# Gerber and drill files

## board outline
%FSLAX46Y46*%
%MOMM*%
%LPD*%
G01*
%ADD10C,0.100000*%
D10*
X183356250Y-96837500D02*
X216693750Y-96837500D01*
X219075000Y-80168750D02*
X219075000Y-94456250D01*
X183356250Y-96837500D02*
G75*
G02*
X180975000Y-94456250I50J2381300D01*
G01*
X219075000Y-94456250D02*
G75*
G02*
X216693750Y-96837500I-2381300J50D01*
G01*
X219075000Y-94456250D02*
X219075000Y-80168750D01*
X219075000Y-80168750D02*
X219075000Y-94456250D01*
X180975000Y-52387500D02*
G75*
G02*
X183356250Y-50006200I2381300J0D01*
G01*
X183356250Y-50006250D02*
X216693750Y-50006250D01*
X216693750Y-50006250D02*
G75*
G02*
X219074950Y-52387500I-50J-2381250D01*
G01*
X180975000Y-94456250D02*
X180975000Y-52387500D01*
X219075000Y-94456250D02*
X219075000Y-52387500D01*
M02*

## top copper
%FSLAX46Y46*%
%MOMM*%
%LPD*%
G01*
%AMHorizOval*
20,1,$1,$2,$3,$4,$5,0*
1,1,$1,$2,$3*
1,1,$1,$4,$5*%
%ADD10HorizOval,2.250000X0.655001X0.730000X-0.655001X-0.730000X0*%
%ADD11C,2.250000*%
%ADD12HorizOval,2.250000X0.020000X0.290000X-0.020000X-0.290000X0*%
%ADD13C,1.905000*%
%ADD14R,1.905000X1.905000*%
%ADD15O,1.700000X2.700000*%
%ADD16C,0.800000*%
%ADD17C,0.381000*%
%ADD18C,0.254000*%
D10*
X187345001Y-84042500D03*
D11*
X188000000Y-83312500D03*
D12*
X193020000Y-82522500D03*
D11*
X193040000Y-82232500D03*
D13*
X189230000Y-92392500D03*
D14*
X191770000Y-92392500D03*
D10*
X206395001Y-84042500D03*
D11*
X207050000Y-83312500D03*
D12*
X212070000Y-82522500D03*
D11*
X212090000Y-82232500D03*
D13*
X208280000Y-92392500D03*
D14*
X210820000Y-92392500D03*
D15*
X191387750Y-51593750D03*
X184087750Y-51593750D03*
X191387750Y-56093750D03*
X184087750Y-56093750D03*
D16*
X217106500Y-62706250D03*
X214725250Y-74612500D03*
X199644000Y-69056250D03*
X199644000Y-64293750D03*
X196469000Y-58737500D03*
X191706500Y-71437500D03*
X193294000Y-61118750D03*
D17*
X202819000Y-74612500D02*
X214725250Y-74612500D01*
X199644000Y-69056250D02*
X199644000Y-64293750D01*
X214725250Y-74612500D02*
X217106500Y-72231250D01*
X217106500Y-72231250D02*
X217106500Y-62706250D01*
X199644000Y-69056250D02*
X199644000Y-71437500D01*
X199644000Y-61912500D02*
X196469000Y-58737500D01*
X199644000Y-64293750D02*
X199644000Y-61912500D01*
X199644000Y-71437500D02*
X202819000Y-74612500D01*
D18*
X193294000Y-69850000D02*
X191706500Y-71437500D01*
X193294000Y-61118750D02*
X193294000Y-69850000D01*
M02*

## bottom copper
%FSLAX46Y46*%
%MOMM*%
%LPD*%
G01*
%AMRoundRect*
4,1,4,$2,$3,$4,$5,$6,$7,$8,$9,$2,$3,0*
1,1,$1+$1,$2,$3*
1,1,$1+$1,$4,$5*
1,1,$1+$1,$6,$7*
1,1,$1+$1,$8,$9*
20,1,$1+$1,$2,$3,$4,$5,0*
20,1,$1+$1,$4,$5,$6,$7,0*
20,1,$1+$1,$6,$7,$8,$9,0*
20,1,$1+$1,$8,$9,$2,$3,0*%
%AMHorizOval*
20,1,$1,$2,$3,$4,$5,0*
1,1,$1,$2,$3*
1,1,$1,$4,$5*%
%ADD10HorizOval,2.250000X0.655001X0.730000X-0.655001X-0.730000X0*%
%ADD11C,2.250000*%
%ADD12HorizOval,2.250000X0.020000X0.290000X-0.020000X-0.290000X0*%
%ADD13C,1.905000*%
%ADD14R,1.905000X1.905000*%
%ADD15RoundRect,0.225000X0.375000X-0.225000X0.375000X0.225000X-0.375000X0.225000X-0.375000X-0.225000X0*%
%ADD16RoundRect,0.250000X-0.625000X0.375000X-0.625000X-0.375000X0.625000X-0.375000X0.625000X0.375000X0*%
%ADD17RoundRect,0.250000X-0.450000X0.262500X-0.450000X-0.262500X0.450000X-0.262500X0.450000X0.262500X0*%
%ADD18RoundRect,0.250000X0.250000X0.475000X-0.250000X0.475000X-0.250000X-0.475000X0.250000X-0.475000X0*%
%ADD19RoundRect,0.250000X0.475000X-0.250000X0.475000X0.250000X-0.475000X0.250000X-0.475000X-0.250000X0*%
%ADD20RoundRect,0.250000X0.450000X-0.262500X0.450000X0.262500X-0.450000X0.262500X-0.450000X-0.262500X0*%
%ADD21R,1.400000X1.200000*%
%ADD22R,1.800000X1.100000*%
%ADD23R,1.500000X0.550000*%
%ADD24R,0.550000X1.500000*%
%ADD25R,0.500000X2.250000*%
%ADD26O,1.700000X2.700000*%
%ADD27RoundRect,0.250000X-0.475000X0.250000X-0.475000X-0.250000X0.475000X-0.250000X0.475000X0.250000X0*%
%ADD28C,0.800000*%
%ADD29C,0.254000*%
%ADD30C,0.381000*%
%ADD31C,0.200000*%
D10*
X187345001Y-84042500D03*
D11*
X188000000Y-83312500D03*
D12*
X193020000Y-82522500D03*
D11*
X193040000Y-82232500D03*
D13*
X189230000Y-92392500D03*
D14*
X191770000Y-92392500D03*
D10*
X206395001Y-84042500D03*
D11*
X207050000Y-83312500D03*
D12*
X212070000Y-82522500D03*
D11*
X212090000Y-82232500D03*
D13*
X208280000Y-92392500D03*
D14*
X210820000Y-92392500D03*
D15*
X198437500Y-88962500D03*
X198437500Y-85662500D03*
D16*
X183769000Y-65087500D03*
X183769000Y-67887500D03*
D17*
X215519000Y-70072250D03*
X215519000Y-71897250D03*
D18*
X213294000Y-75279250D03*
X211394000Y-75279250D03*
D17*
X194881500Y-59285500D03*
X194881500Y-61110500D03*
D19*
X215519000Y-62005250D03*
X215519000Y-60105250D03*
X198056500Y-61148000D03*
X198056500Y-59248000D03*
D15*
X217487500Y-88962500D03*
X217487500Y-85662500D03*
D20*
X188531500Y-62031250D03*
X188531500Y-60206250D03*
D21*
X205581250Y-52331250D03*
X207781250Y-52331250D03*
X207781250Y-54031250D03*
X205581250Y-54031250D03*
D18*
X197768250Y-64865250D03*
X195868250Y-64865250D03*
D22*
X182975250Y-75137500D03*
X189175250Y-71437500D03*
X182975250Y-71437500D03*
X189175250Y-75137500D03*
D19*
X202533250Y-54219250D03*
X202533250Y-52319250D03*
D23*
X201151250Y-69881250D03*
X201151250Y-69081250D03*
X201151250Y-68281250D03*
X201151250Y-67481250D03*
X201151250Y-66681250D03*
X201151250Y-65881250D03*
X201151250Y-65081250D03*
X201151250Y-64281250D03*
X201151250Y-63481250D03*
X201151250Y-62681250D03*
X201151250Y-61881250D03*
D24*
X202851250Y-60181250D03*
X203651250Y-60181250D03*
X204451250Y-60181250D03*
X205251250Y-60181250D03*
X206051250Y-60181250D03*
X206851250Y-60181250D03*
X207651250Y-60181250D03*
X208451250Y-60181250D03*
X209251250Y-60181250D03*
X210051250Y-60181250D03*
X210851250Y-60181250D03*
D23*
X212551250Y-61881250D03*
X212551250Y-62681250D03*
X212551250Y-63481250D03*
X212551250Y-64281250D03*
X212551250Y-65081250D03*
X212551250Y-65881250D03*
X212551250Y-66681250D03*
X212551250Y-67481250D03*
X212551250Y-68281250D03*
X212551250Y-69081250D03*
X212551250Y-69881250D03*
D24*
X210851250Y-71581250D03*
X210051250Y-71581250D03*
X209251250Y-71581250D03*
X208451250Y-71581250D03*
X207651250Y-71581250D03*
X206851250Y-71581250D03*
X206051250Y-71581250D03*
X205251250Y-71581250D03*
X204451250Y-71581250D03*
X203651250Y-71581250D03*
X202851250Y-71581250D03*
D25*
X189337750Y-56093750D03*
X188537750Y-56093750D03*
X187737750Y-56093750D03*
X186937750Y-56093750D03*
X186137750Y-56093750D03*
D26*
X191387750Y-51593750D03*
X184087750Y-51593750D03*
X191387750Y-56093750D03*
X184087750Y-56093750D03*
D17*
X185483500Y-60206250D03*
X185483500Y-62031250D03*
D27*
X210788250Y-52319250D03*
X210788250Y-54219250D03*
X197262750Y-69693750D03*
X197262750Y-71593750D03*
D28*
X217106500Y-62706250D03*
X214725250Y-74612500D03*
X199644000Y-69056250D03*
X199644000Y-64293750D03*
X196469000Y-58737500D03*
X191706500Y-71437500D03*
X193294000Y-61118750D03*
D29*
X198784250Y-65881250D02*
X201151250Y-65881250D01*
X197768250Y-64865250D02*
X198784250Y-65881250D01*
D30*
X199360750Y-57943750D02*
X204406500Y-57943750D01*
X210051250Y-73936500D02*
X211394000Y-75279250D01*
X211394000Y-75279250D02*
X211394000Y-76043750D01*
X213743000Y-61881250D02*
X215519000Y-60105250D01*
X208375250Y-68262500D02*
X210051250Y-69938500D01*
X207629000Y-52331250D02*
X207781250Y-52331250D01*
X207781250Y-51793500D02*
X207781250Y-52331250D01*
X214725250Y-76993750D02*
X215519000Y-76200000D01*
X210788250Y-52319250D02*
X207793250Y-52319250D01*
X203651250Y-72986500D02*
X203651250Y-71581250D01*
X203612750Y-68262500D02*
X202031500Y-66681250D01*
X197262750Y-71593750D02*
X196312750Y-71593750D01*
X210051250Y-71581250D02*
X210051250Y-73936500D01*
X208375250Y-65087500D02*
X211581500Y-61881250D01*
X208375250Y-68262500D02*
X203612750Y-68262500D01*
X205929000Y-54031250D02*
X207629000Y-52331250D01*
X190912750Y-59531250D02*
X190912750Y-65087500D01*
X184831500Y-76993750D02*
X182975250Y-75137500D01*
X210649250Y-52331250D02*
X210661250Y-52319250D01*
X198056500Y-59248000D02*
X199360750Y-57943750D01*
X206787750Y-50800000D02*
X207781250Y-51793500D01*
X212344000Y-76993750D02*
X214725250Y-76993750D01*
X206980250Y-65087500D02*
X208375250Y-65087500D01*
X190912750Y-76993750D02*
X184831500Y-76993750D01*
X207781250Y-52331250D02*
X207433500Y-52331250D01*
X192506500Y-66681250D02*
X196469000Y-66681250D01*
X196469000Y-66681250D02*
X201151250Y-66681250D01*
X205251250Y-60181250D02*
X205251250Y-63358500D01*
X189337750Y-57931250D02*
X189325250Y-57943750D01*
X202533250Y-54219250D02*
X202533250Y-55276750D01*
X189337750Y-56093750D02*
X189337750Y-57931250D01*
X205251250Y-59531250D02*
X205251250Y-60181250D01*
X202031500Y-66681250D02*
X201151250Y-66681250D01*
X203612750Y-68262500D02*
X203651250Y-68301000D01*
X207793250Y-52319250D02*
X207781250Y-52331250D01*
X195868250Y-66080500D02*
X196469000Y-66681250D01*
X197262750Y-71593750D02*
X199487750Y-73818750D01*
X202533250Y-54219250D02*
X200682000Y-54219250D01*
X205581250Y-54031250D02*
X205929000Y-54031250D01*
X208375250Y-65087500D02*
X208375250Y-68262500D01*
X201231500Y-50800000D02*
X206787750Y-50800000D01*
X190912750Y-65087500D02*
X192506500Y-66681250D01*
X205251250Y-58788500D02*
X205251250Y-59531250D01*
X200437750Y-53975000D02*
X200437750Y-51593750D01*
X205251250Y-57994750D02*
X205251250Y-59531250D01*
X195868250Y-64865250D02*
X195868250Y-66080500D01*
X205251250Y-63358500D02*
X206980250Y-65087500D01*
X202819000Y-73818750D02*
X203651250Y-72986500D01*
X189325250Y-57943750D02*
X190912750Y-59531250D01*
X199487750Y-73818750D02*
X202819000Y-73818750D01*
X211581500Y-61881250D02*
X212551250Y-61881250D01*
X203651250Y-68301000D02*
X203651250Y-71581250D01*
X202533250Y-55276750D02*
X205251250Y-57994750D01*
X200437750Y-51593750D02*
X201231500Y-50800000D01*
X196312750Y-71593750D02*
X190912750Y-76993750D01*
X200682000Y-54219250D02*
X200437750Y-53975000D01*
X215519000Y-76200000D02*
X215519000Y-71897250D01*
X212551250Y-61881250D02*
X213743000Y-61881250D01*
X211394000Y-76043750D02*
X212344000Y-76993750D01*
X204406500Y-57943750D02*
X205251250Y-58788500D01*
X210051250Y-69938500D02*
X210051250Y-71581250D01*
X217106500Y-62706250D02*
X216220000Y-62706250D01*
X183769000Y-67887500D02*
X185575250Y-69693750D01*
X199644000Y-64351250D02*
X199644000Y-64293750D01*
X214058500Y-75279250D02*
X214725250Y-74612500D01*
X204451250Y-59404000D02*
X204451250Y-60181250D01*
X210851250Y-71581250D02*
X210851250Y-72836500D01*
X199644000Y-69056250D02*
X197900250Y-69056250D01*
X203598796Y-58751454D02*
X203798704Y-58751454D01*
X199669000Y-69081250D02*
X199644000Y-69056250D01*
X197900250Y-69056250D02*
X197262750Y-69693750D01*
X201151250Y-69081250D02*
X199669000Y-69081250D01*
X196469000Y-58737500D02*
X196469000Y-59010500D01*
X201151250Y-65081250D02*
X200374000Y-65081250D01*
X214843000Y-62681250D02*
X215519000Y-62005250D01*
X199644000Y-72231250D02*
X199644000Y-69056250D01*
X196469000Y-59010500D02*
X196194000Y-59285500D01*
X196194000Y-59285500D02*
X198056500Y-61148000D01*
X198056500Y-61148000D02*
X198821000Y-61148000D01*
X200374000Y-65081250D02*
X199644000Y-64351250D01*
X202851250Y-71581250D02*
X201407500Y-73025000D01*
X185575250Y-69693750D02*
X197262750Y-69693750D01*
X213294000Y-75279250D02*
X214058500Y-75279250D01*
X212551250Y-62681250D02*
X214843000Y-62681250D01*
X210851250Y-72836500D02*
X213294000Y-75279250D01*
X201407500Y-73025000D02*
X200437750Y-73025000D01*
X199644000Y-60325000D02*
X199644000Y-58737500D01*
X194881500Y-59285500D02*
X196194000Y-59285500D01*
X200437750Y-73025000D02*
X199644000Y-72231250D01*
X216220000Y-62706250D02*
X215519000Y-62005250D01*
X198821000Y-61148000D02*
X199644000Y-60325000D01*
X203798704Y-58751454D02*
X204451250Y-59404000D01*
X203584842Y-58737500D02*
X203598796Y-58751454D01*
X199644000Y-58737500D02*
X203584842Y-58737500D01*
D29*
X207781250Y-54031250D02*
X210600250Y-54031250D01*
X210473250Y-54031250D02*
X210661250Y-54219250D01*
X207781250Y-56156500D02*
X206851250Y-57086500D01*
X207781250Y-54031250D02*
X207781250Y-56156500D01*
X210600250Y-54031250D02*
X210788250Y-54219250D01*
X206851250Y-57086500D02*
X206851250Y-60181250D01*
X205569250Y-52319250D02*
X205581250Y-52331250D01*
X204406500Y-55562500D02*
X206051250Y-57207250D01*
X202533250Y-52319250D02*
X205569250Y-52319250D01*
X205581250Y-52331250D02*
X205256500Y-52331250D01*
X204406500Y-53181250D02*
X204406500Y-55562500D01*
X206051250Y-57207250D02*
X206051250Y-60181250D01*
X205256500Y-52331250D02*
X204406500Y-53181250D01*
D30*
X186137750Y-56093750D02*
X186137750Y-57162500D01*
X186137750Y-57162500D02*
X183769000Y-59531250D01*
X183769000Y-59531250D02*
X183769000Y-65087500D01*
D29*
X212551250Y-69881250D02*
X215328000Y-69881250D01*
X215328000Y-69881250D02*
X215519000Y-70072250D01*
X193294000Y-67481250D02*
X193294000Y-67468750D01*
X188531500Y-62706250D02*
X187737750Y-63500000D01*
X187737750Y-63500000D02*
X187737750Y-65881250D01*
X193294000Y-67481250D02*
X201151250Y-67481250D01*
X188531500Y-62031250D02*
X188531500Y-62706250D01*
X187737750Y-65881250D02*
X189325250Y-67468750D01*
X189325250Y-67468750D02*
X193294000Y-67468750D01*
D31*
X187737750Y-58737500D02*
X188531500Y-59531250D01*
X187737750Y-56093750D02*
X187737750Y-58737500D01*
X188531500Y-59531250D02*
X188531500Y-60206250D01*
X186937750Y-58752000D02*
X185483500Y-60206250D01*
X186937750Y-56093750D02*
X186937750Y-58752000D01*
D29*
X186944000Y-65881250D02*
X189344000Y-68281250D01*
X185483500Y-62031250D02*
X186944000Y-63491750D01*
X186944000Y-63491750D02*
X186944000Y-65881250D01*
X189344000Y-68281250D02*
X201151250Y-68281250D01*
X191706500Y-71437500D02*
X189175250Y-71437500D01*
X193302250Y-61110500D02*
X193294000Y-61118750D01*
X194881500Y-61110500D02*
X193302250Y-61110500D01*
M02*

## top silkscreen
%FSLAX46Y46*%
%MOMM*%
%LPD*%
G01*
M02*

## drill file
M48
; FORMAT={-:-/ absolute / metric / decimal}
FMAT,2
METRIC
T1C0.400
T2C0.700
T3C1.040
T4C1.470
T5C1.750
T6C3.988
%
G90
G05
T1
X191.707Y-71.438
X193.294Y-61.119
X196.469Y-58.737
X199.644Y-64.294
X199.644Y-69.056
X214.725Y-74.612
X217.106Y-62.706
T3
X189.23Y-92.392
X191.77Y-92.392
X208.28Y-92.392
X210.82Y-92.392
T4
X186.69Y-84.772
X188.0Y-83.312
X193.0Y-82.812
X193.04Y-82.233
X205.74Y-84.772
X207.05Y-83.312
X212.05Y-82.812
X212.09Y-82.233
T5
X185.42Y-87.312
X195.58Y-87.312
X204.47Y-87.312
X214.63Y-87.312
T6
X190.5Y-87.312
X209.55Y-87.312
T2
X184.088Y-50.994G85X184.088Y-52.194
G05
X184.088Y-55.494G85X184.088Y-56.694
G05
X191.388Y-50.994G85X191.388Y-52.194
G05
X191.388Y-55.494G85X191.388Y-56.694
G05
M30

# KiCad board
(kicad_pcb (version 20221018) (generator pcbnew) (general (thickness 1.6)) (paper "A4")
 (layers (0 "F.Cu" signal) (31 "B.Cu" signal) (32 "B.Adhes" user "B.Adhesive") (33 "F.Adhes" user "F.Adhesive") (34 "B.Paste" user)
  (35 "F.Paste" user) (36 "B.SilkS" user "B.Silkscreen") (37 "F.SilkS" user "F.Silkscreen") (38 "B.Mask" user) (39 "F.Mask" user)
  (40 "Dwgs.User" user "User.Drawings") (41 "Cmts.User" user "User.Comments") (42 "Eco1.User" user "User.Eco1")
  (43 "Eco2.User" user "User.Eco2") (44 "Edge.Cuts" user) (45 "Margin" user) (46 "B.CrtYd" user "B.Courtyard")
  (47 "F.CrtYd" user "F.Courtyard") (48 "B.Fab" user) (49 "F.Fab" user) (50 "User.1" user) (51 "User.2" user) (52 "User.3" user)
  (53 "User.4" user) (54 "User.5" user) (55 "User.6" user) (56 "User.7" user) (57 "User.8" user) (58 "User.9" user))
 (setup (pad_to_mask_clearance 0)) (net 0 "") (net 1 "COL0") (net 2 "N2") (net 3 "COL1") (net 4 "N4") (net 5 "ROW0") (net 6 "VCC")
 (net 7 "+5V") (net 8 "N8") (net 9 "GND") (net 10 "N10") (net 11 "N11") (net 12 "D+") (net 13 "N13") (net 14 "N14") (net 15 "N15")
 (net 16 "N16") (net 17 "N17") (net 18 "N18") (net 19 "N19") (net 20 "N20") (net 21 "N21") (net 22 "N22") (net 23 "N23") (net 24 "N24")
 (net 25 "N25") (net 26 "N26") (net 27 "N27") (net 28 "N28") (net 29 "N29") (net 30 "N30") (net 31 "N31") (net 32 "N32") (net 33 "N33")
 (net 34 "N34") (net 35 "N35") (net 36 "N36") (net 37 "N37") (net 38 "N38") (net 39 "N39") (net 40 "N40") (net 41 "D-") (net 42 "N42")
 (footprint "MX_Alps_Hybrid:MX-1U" (layer "F.Cu") (at 190.5 87.3125)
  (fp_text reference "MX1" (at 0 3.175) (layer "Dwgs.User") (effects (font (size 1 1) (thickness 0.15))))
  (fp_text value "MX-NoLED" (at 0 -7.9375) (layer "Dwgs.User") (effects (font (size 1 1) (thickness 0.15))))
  (pad "" np_thru_hole circle (at -5.08 0 48.0996) (size 1.75 1.75) (drill 1.75) (layers "*.Cu" "*.Mask"))
  (pad "" np_thru_hole circle (at 0 0) (size 3.9878 3.9878) (drill 3.9878) (layers "*.Cu" "*.Mask"))
  (pad "" np_thru_hole circle (at 5.08 0 48.0996) (size 1.75 1.75) (drill 1.75) (layers "*.Cu" "*.Mask"))
  (pad "1" thru_hole oval (at -3.81 -2.54 48.0996) (size 4.211556 2.25) (drill 1.47 (offset 0.980778 0)) (layers "*.Cu" "B.Mask")
   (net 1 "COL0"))
  (pad "1" thru_hole circle (at -2.5 -4) (size 2.25 2.25) (drill 1.47) (layers "*.Cu" "B.Mask") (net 1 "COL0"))
  (pad "2" thru_hole oval (at 2.5 -4.5 86.0548) (size 2.831378 2.25) (drill 1.47 (offset 0.290689 0)) (layers "*.Cu" "B.Mask") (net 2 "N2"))
  (pad "2" thru_hole circle (at 2.54 -5.08) (size 2.25 2.25) (drill 1.47) (layers "*.Cu" "B.Mask") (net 2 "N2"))
  (pad "3" thru_hole circle (at -1.27 5.08) (size 1.905 1.905) (drill 1.04) (layers "*.Cu" "B.Mask"))
  (pad "4" thru_hole rect (at 1.27 5.08) (size 1.905 1.905) (drill 1.04) (layers "*.Cu" "B.Mask")))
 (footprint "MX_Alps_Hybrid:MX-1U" (layer "F.Cu") (at 209.55 87.3125)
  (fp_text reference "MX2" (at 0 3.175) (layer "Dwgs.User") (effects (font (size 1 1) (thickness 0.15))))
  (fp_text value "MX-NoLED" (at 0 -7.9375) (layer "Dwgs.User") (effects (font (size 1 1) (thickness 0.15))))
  (pad "" np_thru_hole circle (at -5.08 0 48.0996) (size 1.75 1.75) (drill 1.75) (layers "*.Cu" "*.Mask"))
  (pad "" np_thru_hole circle (at 0 0) (size 3.9878 3.9878) (drill 3.9878) (layers "*.Cu" "*.Mask"))
  (pad "" np_thru_hole circle (at 5.08 0 48.0996) (size 1.75 1.75) (drill 1.75) (layers "*.Cu" "*.Mask"))
  (pad "1" thru_hole oval (at -3.81 -2.54 48.0996) (size 4.211556 2.25) (drill 1.47 (offset 0.980778 0)) (layers "*.Cu" "B.Mask")
   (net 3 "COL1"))
  (pad "1" thru_hole circle (at -2.5 -4) (size 2.25 2.25) (drill 1.47) (layers "*.Cu" "B.Mask") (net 3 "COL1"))
  (pad "2" thru_hole oval (at 2.5 -4.5 86.0548) (size 2.831378 2.25) (drill 1.47 (offset 0.290689 0)) (layers "*.Cu" "B.Mask") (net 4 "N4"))
  (pad "2" thru_hole circle (at 2.54 -5.08) (size 2.25 2.25) (drill 1.47) (layers "*.Cu" "B.Mask") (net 4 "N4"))
  (pad "3" thru_hole circle (at -1.27 5.08) (size 1.905 1.905) (drill 1.04) (layers "*.Cu" "B.Mask"))
  (pad "4" thru_hole rect (at 1.27 5.08) (size 1.905 1.905) (drill 1.04) (layers "*.Cu" "B.Mask")))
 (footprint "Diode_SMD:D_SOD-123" (layer "B.Cu") (at 198.4375 87.3125 90)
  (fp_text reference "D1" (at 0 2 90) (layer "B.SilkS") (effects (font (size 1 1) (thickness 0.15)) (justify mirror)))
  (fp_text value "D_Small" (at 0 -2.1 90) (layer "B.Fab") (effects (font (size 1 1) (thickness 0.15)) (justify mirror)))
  (pad "1" smd roundrect (at -1.65 0 90) (size 0.9 1.2) (layers "B.Cu" "B.Paste" "B.Mask") (roundrect_rratio 0.25) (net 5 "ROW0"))
  (pad "2" smd roundrect (at 1.65 0 90) (size 0.9 1.2) (layers "B.Cu" "B.Paste" "B.Mask") (roundrect_rratio 0.25) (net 2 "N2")))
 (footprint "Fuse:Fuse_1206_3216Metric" (layer "B.Cu") (at 183.769 66.4875 -90)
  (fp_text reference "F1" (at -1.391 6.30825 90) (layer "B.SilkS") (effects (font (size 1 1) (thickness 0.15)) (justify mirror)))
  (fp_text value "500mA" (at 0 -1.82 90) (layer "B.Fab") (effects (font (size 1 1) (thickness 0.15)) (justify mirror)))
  (pad "1" smd roundrect (at -1.4 0 270) (size 1.25 1.75) (layers "B.Cu" "B.Paste" "B.Mask") (roundrect_rratio 0.2) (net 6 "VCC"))
  (pad "2" smd roundrect (at 1.4 0 270) (size 1.25 1.75) (layers "B.Cu" "B.Paste" "B.Mask") (roundrect_rratio 0.2) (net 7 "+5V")))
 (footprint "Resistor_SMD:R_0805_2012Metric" (layer "B.Cu") (at 215.519 70.98475 -90)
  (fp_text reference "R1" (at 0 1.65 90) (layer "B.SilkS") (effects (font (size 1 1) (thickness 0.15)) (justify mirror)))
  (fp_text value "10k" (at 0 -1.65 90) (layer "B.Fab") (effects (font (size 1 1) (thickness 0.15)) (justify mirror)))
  (pad "1" smd roundrect (at -0.9125 0 270) (size 1.025 1.4) (layers "B.Cu" "B.Paste" "B.Mask") (roundrect_rratio 0.243902) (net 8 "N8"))
  (pad "2" smd roundrect (at 0.9125 0 270) (size 1.025 1.4) (layers "B.Cu" "B.Paste" "B.Mask") (roundrect_rratio 0.243902) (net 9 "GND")))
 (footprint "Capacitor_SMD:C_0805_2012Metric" (layer "B.Cu") (at 212.344 75.27925 180)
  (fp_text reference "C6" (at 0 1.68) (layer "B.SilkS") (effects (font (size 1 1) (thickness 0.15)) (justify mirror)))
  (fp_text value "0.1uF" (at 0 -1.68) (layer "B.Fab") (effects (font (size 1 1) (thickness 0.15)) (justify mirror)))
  (pad "1" smd roundrect (at -0.95 0 180) (size 1 1.45) (layers "B.Cu" "B.Paste" "B.Mask") (roundrect_rratio 0.25) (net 7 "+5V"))
  (pad "2" smd roundrect (at 0.95 0 180) (size 1 1.45) (layers "B.Cu" "B.Paste" "B.Mask") (roundrect_rratio 0.25) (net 9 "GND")))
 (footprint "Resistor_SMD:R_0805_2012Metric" (layer "B.Cu") (at 194.8815 60.198 -90)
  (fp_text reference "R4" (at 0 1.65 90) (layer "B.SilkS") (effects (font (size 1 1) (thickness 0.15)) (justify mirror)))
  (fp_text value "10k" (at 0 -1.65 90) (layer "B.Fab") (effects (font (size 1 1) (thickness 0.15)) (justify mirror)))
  (pad "1" smd roundrect (at -0.9125 0 270) (size 1.025 1.4) (layers "B.Cu" "B.Paste" "B.Mask") (roundrect_rratio 0.243902) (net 7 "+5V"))
  (pad "2" smd roundrect (at 0.9125 0 270) (size 1.025 1.4) (layers "B.Cu" "B.Paste" "B.Mask") (roundrect_rratio 0.243902) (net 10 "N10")))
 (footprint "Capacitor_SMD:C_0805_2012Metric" (layer "B.Cu") (at 215.519 61.05525 90)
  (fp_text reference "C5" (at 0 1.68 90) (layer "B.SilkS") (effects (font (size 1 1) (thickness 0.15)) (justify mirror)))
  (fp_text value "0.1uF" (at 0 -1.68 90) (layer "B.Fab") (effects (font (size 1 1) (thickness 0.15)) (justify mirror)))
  (pad "1" smd roundrect (at -0.95 0 90) (size 1 1.45) (layers "B.Cu" "B.Paste" "B.Mask") (roundrect_rratio 0.25) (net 7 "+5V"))
  (pad "2" smd roundrect (at 0.95 0 90) (size 1 1.45) (layers "B.Cu" "B.Paste" "B.Mask") (roundrect_rratio 0.25) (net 9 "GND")))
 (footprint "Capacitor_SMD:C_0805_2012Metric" (layer "B.Cu") (at 198.0565 60.198 90)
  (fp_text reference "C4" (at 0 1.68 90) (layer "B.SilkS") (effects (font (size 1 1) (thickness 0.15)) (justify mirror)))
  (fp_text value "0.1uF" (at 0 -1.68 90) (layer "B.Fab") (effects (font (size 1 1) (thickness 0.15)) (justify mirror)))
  (pad "1" smd roundrect (at -0.95 0 90) (size 1 1.45) (layers "B.Cu" "B.Paste" "B.Mask") (roundrect_rratio 0.25) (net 7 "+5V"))
  (pad "2" smd roundrect (at 0.95 0 90) (size 1 1.45) (layers "B.Cu" "B.Paste" "B.Mask") (roundrect_rratio 0.25) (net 9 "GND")))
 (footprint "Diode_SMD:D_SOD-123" (layer "B.Cu") (at 217.4875 87.3125 90)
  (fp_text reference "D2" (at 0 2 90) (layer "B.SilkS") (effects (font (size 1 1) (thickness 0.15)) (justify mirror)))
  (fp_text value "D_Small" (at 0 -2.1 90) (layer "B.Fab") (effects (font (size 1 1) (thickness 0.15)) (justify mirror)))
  (pad "1" smd roundrect (at -1.65 0 90) (size 0.9 1.2) (layers "B.Cu" "B.Paste" "B.Mask") (roundrect_rratio 0.25) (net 5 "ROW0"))
  (pad "2" smd roundrect (at 1.65 0 90) (size 0.9 1.2) (layers "B.Cu" "B.Paste" "B.Mask") (roundrect_rratio 0.25) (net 4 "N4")))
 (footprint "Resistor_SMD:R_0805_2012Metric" (layer "B.Cu") (at 188.5315 61.11875 90)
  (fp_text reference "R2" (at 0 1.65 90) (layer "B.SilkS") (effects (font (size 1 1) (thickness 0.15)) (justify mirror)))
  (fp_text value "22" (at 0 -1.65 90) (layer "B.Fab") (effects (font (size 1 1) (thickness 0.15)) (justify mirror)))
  (pad "1" smd roundrect (at -0.9125 0 90) (size 1.025 1.4) (layers "B.Cu" "B.Paste" "B.Mask") (roundrect_rratio 0.243902) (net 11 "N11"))
  (pad "2" smd roundrect (at 0.9125 0 90) (size 1.025 1.4) (layers "B.Cu" "B.Paste" "B.Mask") (roundrect_rratio 0.243902) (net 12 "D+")))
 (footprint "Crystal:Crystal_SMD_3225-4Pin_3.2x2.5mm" (layer "B.Cu") (at 206.68125 53.18125)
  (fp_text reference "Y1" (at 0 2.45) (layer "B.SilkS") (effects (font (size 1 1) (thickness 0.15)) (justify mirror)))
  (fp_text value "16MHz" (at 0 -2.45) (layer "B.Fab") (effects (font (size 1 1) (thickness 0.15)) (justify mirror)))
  (pad "1" smd rect (at -1.1 -0.85) (size 1.4 1.2) (layers "B.Cu" "B.Paste" "B.Mask") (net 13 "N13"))
  (pad "2" smd rect (at 1.1 -0.85) (size 1.4 1.2) (layers "B.Cu" "B.Paste" "B.Mask") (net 9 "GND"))
  (pad "3" smd rect (at 1.1 0.85) (size 1.4 1.2) (layers "B.Cu" "B.Paste" "B.Mask") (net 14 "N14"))
  (pad "4" smd rect (at -1.1 0.85) (size 1.4 1.2) (layers "B.Cu" "B.Paste" "B.Mask") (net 9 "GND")))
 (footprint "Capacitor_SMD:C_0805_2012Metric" (layer "B.Cu") (at 196.81825 64.86525 180)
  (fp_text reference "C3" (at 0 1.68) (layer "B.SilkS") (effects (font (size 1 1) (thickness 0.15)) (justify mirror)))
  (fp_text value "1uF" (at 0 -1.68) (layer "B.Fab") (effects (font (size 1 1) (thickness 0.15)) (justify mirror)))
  (pad "1" smd roundrect (at -0.95 0 180) (size 1 1.45) (layers "B.Cu" "B.Paste" "B.Mask") (roundrect_rratio 0.25) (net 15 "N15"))
  (pad "2" smd roundrect (at 0.95 0 180) (size 1 1.45) (layers "B.Cu" "B.Paste" "B.Mask") (roundrect_rratio 0.25) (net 9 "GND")))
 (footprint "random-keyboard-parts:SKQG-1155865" (layer "B.Cu") (at 186.07525 73.2875 180)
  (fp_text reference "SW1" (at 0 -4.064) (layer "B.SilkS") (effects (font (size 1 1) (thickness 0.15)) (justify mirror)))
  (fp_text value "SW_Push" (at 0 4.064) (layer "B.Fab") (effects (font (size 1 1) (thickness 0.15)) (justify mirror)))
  (pad "1" smd rect (at 3.1 -1.85 180) (size 1.8 1.1) (layers "B.Cu" "B.Paste" "B.Mask") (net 9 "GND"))
  (pad "2" smd rect (at -3.1 1.85 180) (size 1.8 1.1) (layers "B.Cu" "B.Paste" "B.Mask") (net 10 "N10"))
  (pad "3" smd rect (at 3.1 1.85 180) (size 1.8 1.1) (layers "B.Cu" "B.Paste" "B.Mask"))
  (pad "4" smd rect (at -3.1 -1.85 180) (size 1.8 1.1) (layers "B.Cu" "B.Paste" "B.Mask")))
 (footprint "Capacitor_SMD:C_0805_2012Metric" (layer "B.Cu") (at 202.53325 53.26925 90)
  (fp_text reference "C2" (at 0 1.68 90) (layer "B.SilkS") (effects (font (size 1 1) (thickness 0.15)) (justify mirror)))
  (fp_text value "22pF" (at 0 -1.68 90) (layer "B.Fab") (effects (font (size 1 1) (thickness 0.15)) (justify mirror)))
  (pad "1" smd roundrect (at -0.95 0 90) (size 1 1.45) (layers "B.Cu" "B.Paste" "B.Mask") (roundrect_rratio 0.25) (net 9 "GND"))
  (pad "2" smd roundrect (at 0.95 0 90) (size 1 1.45) (layers "B.Cu" "B.Paste" "B.Mask") (roundrect_rratio 0.25) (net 13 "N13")))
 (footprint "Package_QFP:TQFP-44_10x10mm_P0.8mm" (layer "B.Cu") (at 206.85125 65.88125)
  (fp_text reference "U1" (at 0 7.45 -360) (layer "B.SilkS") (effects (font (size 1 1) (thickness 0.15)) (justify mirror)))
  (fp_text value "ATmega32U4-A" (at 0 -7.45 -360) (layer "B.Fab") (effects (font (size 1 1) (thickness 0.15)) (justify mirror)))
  (pad "1" smd rect (at -5.7 4) (size 1.5 0.55) (layers "B.Cu" "B.Paste" "B.Mask") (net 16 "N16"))
  (pad "2" smd rect (at -5.7 3.2) (size 1.5 0.55) (layers "B.Cu" "B.Paste" "B.Mask") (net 7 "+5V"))
  (pad "3" smd rect (at -5.7 2.4) (size 1.5 0.55) (layers "B.Cu" "B.Paste" "B.Mask") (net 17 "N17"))
  (pad "4" smd rect (at -5.7 1.6) (size 1.5 0.55) (layers "B.Cu" "B.Paste" "B.Mask") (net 11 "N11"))
  (pad "5" smd rect (at -5.7 0.8) (size 1.5 0.55) (layers "B.Cu" "B.Paste" "B.Mask") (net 9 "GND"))
  (pad "6" smd rect (at -5.7 0) (size 1.5 0.55) (layers "B.Cu" "B.Paste" "B.Mask") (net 15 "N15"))
  (pad "7" smd rect (at -5.7 -0.8) (size 1.5 0.55) (layers "B.Cu" "B.Paste" "B.Mask") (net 7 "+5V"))
  (pad "8" smd rect (at -5.7 -1.6) (size 1.5 0.55) (layers "B.Cu" "B.Paste" "B.Mask") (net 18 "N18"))
  (pad "9" smd rect (at -5.7 -2.4) (size 1.5 0.55) (layers "B.Cu" "B.Paste" "B.Mask") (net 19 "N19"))
  (pad "10" smd rect (at -5.7 -3.2) (size 1.5 0.55) (layers "B.Cu" "B.Paste" "B.Mask") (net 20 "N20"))
  (pad "11" smd rect (at -5.7 -4) (size 1.5 0.55) (layers "B.Cu" "B.Paste" "B.Mask") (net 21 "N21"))
  (pad "12" smd rect (at -4 -5.7 270) (size 1.5 0.55) (layers "B.Cu" "B.Paste" "B.Mask") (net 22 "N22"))
  (pad "13" smd rect (at -3.2 -5.7 270) (size 1.5 0.55) (layers "B.Cu" "B.Paste" "B.Mask") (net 10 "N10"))
  (pad "14" smd rect (at -2.4 -5.7 270) (size 1.5 0.55) (layers "B.Cu" "B.Paste" "B.Mask") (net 7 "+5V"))
  (pad "15" smd rect (at -1.6 -5.7 270) (size 1.5 0.55) (layers "B.Cu" "B.Paste" "B.Mask") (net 9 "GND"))
  (pad "16" smd rect (at -0.8 -5.7 270) (size 1.5 0.55) (layers "B.Cu" "B.Paste" "B.Mask") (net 13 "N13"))
  (pad "17" smd rect (at 0 -5.7 270) (size 1.5 0.55) (layers "B.Cu" "B.Paste" "B.Mask") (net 14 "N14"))
  (pad "18" smd rect (at 0.8 -5.7 270) (size 1.5 0.55) (layers "B.Cu" "B.Paste" "B.Mask") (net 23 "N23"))
  (pad "19" smd rect (at 1.6 -5.7 270) (size 1.5 0.55) (layers "B.Cu" "B.Paste" "B.Mask") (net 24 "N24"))
  (pad "20" smd rect (at 2.4 -5.7 270) (size 1.5 0.55) (layers "B.Cu" "B.Paste" "B.Mask") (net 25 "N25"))
  (pad "21" smd rect (at 3.2 -5.7 270) (size 1.5 0.55) (layers "B.Cu" "B.Paste" "B.Mask") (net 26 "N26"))
  (pad "22" smd rect (at 4 -5.7 270) (size 1.5 0.55) (layers "B.Cu" "B.Paste" "B.Mask") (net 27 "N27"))
  (pad "23" smd rect (at 5.7 -4) (size 1.5 0.55) (layers "B.Cu" "B.Paste" "B.Mask") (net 9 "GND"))
  (pad "24" smd rect (at 5.7 -3.2) (size 1.5 0.55) (layers "B.Cu" "B.Paste" "B.Mask") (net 7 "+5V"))
  (pad "25" smd rect (at 5.7 -2.4) (size 1.5 0.55) (layers "B.Cu" "B.Paste" "B.Mask") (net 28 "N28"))
  (pad "26" smd rect (at 5.7 -1.6) (size 1.5 0.55) (layers "B.Cu" "B.Paste" "B.Mask") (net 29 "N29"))
  (pad "27" smd rect (at 5.7 -0.8) (size 1.5 0.55) (layers "B.Cu" "B.Paste" "B.Mask") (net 5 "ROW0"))
  (pad "28" smd rect (at 5.7 0) (size 1.5 0.55) (layers "B.Cu" "B.Paste" "B.Mask") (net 3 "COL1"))
  (pad "29" smd rect (at 5.7 0.8) (size 1.5 0.55) (layers "B.Cu" "B.Paste" "B.Mask") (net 1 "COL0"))
  (pad "30" smd rect (at 5.7 1.6) (size 1.5 0.55) (layers "B.Cu" "B.Paste" "B.Mask") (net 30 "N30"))
  (pad "31" smd rect (at 5.7 2.4) (size 1.5 0.55) (layers "B.Cu" "B.Paste" "B.Mask") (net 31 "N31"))
  (pad "32" smd rect (at 5.7 3.2) (size 1.5 0.55) (layers "B.Cu" "B.Paste" "B.Mask") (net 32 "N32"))
  (pad "33" smd rect (at 5.7 4) (size 1.5 0.55) (layers "B.Cu" "B.Paste" "B.Mask") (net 8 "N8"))
  (pad "34" smd rect (at 4 5.7 270) (size 1.5 0.55) (layers "B.Cu" "B.Paste" "B.Mask") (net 7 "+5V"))
  (pad "35" smd rect (at 3.2 5.7 270) (size 1.5 0.55) (layers "B.Cu" "B.Paste" "B.Mask") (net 9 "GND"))
  (pad "36" smd rect (at 2.4 5.7 270) (size 1.5 0.55) (layers "B.Cu" "B.Paste" "B.Mask") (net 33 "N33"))
  (pad "37" smd rect (at 1.6 5.7 270) (size 1.5 0.55) (layers "B.Cu" "B.Paste" "B.Mask") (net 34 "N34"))
  (pad "38" smd rect (at 0.8 5.7 270) (size 1.5 0.55) (layers "B.Cu" "B.Paste" "B.Mask") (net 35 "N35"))
  (pad "39" smd rect (at 0 5.7 270) (size 1.5 0.55) (layers "B.Cu" "B.Paste" "B.Mask") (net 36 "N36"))
  (pad "40" smd rect (at -0.8 5.7 270) (size 1.5 0.55) (layers "B.Cu" "B.Paste" "B.Mask") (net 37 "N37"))
  (pad "41" smd rect (at -1.6 5.7 270) (size 1.5 0.55) (layers "B.Cu" "B.Paste" "B.Mask") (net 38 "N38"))
  (pad "42" smd rect (at -2.4 5.7 270) (size 1.5 0.55) (layers "B.Cu" "B.Paste" "B.Mask") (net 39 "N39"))
  (pad "43" smd rect (at -3.2 5.7 270) (size 1.5 0.55) (layers "B.Cu" "B.Paste" "B.Mask") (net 9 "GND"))
  (pad "44" smd rect (at -4 5.7 270) (size 1.5 0.55) (layers "B.Cu" "B.Paste" "B.Mask") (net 7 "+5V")))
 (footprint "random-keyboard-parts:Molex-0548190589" (layer "B.Cu") (at 187.73775 51.59375 -90)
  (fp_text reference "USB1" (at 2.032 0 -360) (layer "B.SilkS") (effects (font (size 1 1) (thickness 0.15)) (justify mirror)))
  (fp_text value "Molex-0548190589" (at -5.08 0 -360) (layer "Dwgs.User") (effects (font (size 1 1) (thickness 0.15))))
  (pad "1" smd rect (at 4.5 -1.6 270) (size 2.25 0.5) (layers "B.Cu" "B.Paste" "B.Mask") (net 9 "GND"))
  (pad "2" smd rect (at 4.5 -0.8 270) (size 2.25 0.5) (layers "B.Cu" "B.Paste" "B.Mask") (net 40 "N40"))
  (pad "3" smd rect (at 4.5 0 270) (size 2.25 0.5) (layers "B.Cu" "B.Paste" "B.Mask") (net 12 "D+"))
  (pad "4" smd rect (at 4.5 0.8 270) (size 2.25 0.5) (layers "B.Cu" "B.Paste" "B.Mask") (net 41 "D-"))
  (pad "5" smd rect (at 4.5 1.6 270) (size 2.25 0.5) (layers "B.Cu" "B.Paste" "B.Mask") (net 6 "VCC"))
  (pad "6" thru_hole oval (at 0 -3.65 270) (size 2.7 1.7) (drill oval 1.9 0.7) (layers "*.Cu" "*.Mask") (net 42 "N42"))
  (pad "6" thru_hole oval (at 0 3.65 270) (size 2.7 1.7) (drill oval 1.9 0.7) (layers "*.Cu" "*.Mask") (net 42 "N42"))
  (pad "6" thru_hole oval (at 4.5 -3.65 270) (size 2.7 1.7) (drill oval 1.9 0.7) (layers "*.Cu" "*.Mask") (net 42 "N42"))
  (pad "6" thru_hole oval (at 4.5 3.65 270) (size 2.7 1.7) (drill oval 1.9 0.7) (layers "*.Cu" "*.Mask") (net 42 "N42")))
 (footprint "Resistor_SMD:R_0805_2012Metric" (layer "B.Cu") (at 185.4835 61.11875 -90)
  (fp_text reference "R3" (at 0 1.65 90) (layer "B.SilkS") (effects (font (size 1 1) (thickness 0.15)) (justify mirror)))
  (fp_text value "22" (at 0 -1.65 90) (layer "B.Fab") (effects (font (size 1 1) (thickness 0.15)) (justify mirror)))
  (pad "1" smd roundrect (at -0.9125 0 270) (size 1.025 1.4) (layers "B.Cu" "B.Paste" "B.Mask") (roundrect_rratio 0.243902) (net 41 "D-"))
  (pad "2" smd roundrect (at 0.9125 0 270) (size 1.025 1.4) (layers "B.Cu" "B.Paste" "B.Mask") (roundrect_rratio 0.243902) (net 17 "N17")))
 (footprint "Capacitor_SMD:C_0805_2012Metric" (layer "B.Cu") (at 210.78825 53.26925 -90)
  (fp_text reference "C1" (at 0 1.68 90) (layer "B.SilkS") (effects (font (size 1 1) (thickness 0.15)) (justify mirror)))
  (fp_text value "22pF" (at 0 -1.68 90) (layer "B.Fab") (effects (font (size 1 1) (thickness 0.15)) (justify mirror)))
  (pad "1" smd roundrect (at -0.95 0 270) (size 1 1.45) (layers "B.Cu" "B.Paste" "B.Mask") (roundrect_rratio 0.25) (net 9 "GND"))
  (pad "2" smd roundrect (at 0.95 0 270) (size 1 1.45) (layers "B.Cu" "B.Paste" "B.Mask") (roundrect_rratio 0.25) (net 14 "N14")))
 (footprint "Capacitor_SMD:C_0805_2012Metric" (layer "B.Cu") (at 197.26275 70.64375 -90)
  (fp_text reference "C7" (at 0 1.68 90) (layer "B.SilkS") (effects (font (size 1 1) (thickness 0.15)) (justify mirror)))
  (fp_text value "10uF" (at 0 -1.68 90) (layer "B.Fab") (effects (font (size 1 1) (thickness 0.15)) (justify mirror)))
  (pad "1" smd roundrect (at -0.95 0 270) (size 1 1.45) (layers "B.Cu" "B.Paste" "B.Mask") (roundrect_rratio 0.25) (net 7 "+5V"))
  (pad "2" smd roundrect (at 0.95 0 270) (size 1 1.45) (layers "B.Cu" "B.Paste" "B.Mask") (roundrect_rratio 0.25) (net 9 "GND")))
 (gr_line (start 183.35625 96.8375) (end 216.69375 96.8375) (stroke (width 0.1) (type default)) (layer "Edge.Cuts"))
 (gr_line (start 219.075 80.16875) (end 219.075 94.45625) (stroke (width 0.1) (type default)) (layer "Edge.Cuts"))
 (gr_arc (start 183.35625 96.8375) (mid 181.672452 96.140048) (end 180.975 94.45625) (stroke (width 0.1) (type default)) (layer "Edge.Cuts"))
 (gr_arc (start 219.075 94.45625) (mid 218.377548 96.140048) (end 216.69375 96.8375) (stroke (width 0.1) (type default)) (layer "Edge.Cuts"))
 (gr_line (start 219.075 94.45625) (end 219.075 80.16875) (stroke (width 0.1) (type default)) (layer "Edge.Cuts"))
 (gr_line (start 219.075 80.16875) (end 219.075 94.45625) (stroke (width 0.1) (type default)) (layer "Edge.Cuts"))
 (gr_arc (start 180.975 52.3875) (mid 181.672452 50.703702) (end 183.35625 50.00625) (stroke (width 0.1) (type default)) (layer "Edge.Cuts"))
 (gr_line (start 183.35625 50.00625) (end 216.69375 50.00625) (stroke (width 0.1) (type default)) (layer "Edge.Cuts"))
 (gr_arc (start 216.69375 50.00625) (mid 218.377548 50.703702) (end 219.075 52.3875) (stroke (width 0.1) (type default)) (layer "Edge.Cuts"))
 (gr_line (start 180.975 94.45625) (end 180.975 52.3875) (stroke (width 0.1) (type default)) (layer "Edge.Cuts"))
 (gr_line (start 219.075 94.45625) (end 219.075 52.3875) (stroke (width 0.1) (type default)) (layer "Edge.Cuts"))
 (segment (start 198.78425 65.88125) (end 201.15125 65.88125) (width 0.254) (layer "B.Cu") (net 15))
 (segment (start 197.76825 64.86525) (end 198.78425 65.88125) (width 0.254) (layer "B.Cu") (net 15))
 (segment (start 199.36075 57.94375) (end 204.4065 57.94375) (width 0.381) (layer "B.Cu") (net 9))
 (segment (start 210.05125 73.9365) (end 211.394 75.27925) (width 0.381) (layer "B.Cu") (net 9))
 (segment (start 211.394 75.27925) (end 211.394 76.04375) (width 0.381) (layer "B.Cu") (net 9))
 (segment (start 213.743 61.88125) (end 215.519 60.10525) (width 0.381) (layer "B.Cu") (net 9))
 (segment (start 208.37525 68.2625) (end 210.05125 69.9385) (width 0.381) (layer "B.Cu") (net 9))
 (segment (start 207.629 52.33125) (end 207.78125 52.33125) (width 0.381) (layer "B.Cu") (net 9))
 (segment (start 207.78125 51.7935) (end 207.78125 52.33125) (width 0.381) (layer "B.Cu") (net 9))
 (segment (start 214.72525 76.99375) (end 215.519 76.2) (width 0.381) (layer "B.Cu") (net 9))
 (segment (start 210.78825 52.31925) (end 207.79325 52.31925) (width 0.381) (layer "B.Cu") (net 9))
 (segment (start 203.65125 72.9865) (end 203.65125 71.58125) (width 0.381) (layer "B.Cu") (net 9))
 (segment (start 203.61275 68.2625) (end 202.0315 66.68125) (width 0.381) (layer "B.Cu") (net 9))
 (segment (start 197.26275 71.59375) (end 196.31275 71.59375) (width 0.381) (layer "B.Cu") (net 9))
 (segment (start 210.05125 71.58125) (end 210.05125 73.9365) (width 0.381) (layer "B.Cu") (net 9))
 (segment (start 208.37525 65.0875) (end 211.5815 61.88125) (width 0.381) (layer "B.Cu") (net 9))
 (segment (start 208.37525 68.2625) (end 203.61275 68.2625) (width 0.381) (layer "B.Cu") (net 9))
 (segment (start 205.929 54.03125) (end 207.629 52.33125) (width 0.381) (layer "B.Cu") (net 9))
 (segment (start 190.91275 59.53125) (end 190.91275 65.0875) (width 0.381) (layer "B.Cu") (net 9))
 (segment (start 184.8315 76.99375) (end 182.97525 75.1375) (width 0.381) (layer "B.Cu") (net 9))
 (segment (start 210.64925 52.33125) (end 210.66125 52.31925) (width 0.381) (layer "B.Cu") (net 9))
 (segment (start 198.0565 59.248) (end 199.36075 57.94375) (width 0.381) (layer "B.Cu") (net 9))
 (segment (start 206.78775 50.8) (end 207.78125 51.7935) (width 0.381) (layer "B.Cu") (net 9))
 (segment (start 212.344 76.99375) (end 214.72525 76.99375) (width 0.381) (layer "B.Cu") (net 9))
 (segment (start 206.98025 65.0875) (end 208.37525 65.0875) (width 0.381) (layer "B.Cu") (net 9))
 (segment (start 190.91275 76.99375) (end 184.8315 76.99375) (width 0.381) (layer "B.Cu") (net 9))
 (segment (start 207.78125 52.33125) (end 207.4335 52.33125) (width 0.381) (layer "B.Cu") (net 9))
 (segment (start 192.5065 66.68125) (end 196.469 66.68125) (width 0.381) (layer "B.Cu") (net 9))
 (segment (start 196.469 66.68125) (end 201.15125 66.68125) (width 0.381) (layer "B.Cu") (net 9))
 (segment (start 205.25125 60.18125) (end 205.25125 63.3585) (width 0.381) (layer "B.Cu") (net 9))
 (segment (start 189.33775 57.93125) (end 189.32525 57.94375) (width 0.381) (layer "B.Cu") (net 9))
 (segment (start 202.53325 54.21925) (end 202.53325 55.27675) (width 0.381) (layer "B.Cu") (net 9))
 (segment (start 189.33775 56.09375) (end 189.33775 57.93125) (width 0.381) (layer "B.Cu") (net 9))
 (segment (start 205.25125 59.53125) (end 205.25125 60.18125) (width 0.381) (layer "B.Cu") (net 9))
 (segment (start 202.0315 66.68125) (end 201.15125 66.68125) (width 0.381) (layer "B.Cu") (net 9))
 (segment (start 203.61275 68.2625) (end 203.65125 68.301) (width 0.381) (layer "B.Cu") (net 9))
 (segment (start 207.79325 52.31925) (end 207.78125 52.33125) (width 0.381) (layer "B.Cu") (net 9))
 (segment (start 195.86825 66.0805) (end 196.469 66.68125) (width 0.381) (layer "B.Cu") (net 9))
 (segment (start 197.26275 71.59375) (end 199.48775 73.81875) (width 0.381) (layer "B.Cu") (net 9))
 (segment (start 202.53325 54.21925) (end 200.682 54.21925) (width 0.381) (layer "B.Cu") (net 9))
 (segment (start 205.58125 54.03125) (end 205.929 54.03125) (width 0.381) (layer "B.Cu") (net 9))
 (segment (start 208.37525 65.0875) (end 208.37525 68.2625) (width 0.381) (layer "B.Cu") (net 9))
 (segment (start 201.2315 50.8) (end 206.78775 50.8) (width 0.381) (layer "B.Cu") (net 9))
 (segment (start 190.91275 65.0875) (end 192.5065 66.68125) (width 0.381) (layer "B.Cu") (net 9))
 (segment (start 205.25125 58.7885) (end 205.25125 59.53125) (width 0.381) (layer "B.Cu") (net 9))
 (segment (start 200.43775 53.975) (end 200.43775 51.59375) (width 0.381) (layer "B.Cu") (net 9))
 (segment (start 205.25125 57.99475) (end 205.25125 59.53125) (width 0.381) (layer "B.Cu") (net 9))
 (segment (start 195.86825 64.86525) (end 195.86825 66.0805) (width 0.381) (layer "B.Cu") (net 9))
 (segment (start 205.25125 63.3585) (end 206.98025 65.0875) (width 0.381) (layer "B.Cu") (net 9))
 (segment (start 202.819 73.81875) (end 203.65125 72.9865) (width 0.381) (layer "B.Cu") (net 9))
 (segment (start 189.32525 57.94375) (end 190.91275 59.53125) (width 0.381) (layer "B.Cu") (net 9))
 (segment (start 199.48775 73.81875) (end 202.819 73.81875) (width 0.381) (layer "B.Cu") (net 9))
 (segment (start 211.5815 61.88125) (end 212.55125 61.88125) (width 0.381) (layer "B.Cu") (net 9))
 (segment (start 203.65125 68.301) (end 203.65125 71.58125) (width 0.381) (layer "B.Cu") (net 9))
 (segment (start 202.53325 55.27675) (end 205.25125 57.99475) (width 0.381) (layer "B.Cu") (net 9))
 (segment (start 200.43775 51.59375) (end 201.2315 50.8) (width 0.381) (layer "B.Cu") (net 9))
 (segment (start 196.31275 71.59375) (end 190.91275 76.99375) (width 0.381) (layer "B.Cu") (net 9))
 (segment (start 200.682 54.21925) (end 200.43775 53.975) (width 0.381) (layer "B.Cu") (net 9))
 (segment (start 215.519 76.2) (end 215.519 71.89725) (width 0.381) (layer "B.Cu") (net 9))
 (segment (start 212.55125 61.88125) (end 213.743 61.88125) (width 0.381) (layer "B.Cu") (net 9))
 (segment (start 211.394 76.04375) (end 212.344 76.99375) (width 0.381) (layer "B.Cu") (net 9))
 (segment (start 204.4065 57.94375) (end 205.25125 58.7885) (width 0.381) (layer "B.Cu") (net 9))
 (segment (start 210.05125 69.9385) (end 210.05125 71.58125) (width 0.381) (layer "B.Cu") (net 9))
 (segment (start 202.819 74.6125) (end 214.72525 74.6125) (width 0.381) (layer "F.Cu") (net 7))
 (segment (start 199.644 69.05625) (end 199.644 64.29375) (width 0.381) (layer "F.Cu") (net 7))
 (segment (start 214.72525 74.6125) (end 217.1065 72.23125) (width 0.381) (layer "F.Cu") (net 7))
 (segment (start 217.1065 72.23125) (end 217.1065 62.70625) (width 0.381) (layer "F.Cu") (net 7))
 (segment (start 199.644 69.05625) (end 199.644 71.4375) (width 0.381) (layer "F.Cu") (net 7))
 (segment (start 199.644 61.9125) (end 196.469 58.7375) (width 0.381) (layer "F.Cu") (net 7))
 (segment (start 199.644 64.29375) (end 199.644 61.9125) (width 0.381) (layer "F.Cu") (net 7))
 (segment (start 199.644 71.4375) (end 202.819 74.6125) (width 0.381) (layer "F.Cu") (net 7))
 (via (at 217.1065 62.70625) (size 0.8) (drill 0.4) (layers "F.Cu" "B.Cu") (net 7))
 (via (at 214.72525 74.6125) (size 0.8) (drill 0.4) (layers "F.Cu" "B.Cu") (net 7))
 (via (at 199.644 69.05625) (size 0.8) (drill 0.4) (layers "F.Cu" "B.Cu") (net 7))
 (via (at 199.644 64.29375) (size 0.8) (drill 0.4) (layers "F.Cu" "B.Cu") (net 7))
 (via (at 196.469 58.7375) (size 0.8) (drill 0.4) (layers "F.Cu" "B.Cu") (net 7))
 (segment (start 217.1065 62.70625) (end 216.22 62.70625) (width 0.381) (layer "B.Cu") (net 7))
 (segment (start 183.769 67.8875) (end 185.57525 69.69375) (width 0.381) (layer "B.Cu") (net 7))
 (segment (start 199.644 64.35125) (end 199.644 64.29375) (width 0.381) (layer "B.Cu") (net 7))
 (segment (start 214.0585 75.27925) (end 214.72525 74.6125) (width 0.381) (layer "B.Cu") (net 7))
 (segment (start 204.45125 59.404) (end 204.45125 60.18125) (width 0.381) (layer "B.Cu") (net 7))
 (segment (start 210.85125 71.58125) (end 210.85125 72.8365) (width 0.381) (layer "B.Cu") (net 7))
 (segment (start 199.644 69.05625) (end 197.90025 69.05625) (width 0.381) (layer "B.Cu") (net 7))
 (segment (start 203.598796 58.751454) (end 203.798704 58.751454) (width 0.381) (layer "B.Cu") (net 7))
 (segment (start 199.669 69.08125) (end 199.644 69.05625) (width 0.381) (layer "B.Cu") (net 7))
 (segment (start 197.90025 69.05625) (end 197.26275 69.69375) (width 0.381) (layer "B.Cu") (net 7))
 (segment (start 201.15125 69.08125) (end 199.669 69.08125) (width 0.381) (layer "B.Cu") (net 7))
 (segment (start 196.469 58.7375) (end 196.469 59.0105) (width 0.381) (layer "B.Cu") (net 7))
 (segment (start 201.15125 65.08125) (end 200.374 65.08125) (width 0.381) (layer "B.Cu") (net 7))
 (segment (start 214.843 62.68125) (end 215.519 62.00525) (width 0.381) (layer "B.Cu") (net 7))
 (segment (start 199.644 72.23125) (end 199.644 69.05625) (width 0.381) (layer "B.Cu") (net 7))
 (segment (start 196.469 59.0105) (end 196.194 59.2855) (width 0.381) (layer "B.Cu") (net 7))
 (segment (start 196.194 59.2855) (end 198.0565 61.148) (width 0.381) (layer "B.Cu") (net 7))
 (segment (start 198.0565 61.148) (end 198.821 61.148) (width 0.381) (layer "B.Cu") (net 7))
 (segment (start 200.374 65.08125) (end 199.644 64.35125) (width 0.381) (layer "B.Cu") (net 7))
 (segment (start 202.85125 71.58125) (end 201.4075 73.025) (width 0.381) (layer "B.Cu") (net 7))
 (segment (start 185.57525 69.69375) (end 197.26275 69.69375) (width 0.381) (layer "B.Cu") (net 7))
 (segment (start 213.294 75.27925) (end 214.0585 75.27925) (width 0.381) (layer "B.Cu") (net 7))
 (segment (start 212.55125 62.68125) (end 214.843 62.68125) (width 0.381) (layer "B.Cu") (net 7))
 (segment (start 210.85125 72.8365) (end 213.294 75.27925) (width 0.381) (layer "B.Cu") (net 7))
 (segment (start 201.4075 73.025) (end 200.43775 73.025) (width 0.381) (layer "B.Cu") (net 7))
 (segment (start 199.644 60.325) (end 199.644 58.7375) (width 0.381) (layer "B.Cu") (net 7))
 (segment (start 194.8815 59.2855) (end 196.194 59.2855) (width 0.381) (layer "B.Cu") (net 7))
 (segment (start 200.43775 73.025) (end 199.644 72.23125) (width 0.381) (layer "B.Cu") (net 7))
 (segment (start 216.22 62.70625) (end 215.519 62.00525) (width 0.381) (layer "B.Cu") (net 7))
 (segment (start 198.821 61.148) (end 199.644 60.325) (width 0.381) (layer "B.Cu") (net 7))
 (segment (start 203.798704 58.751454) (end 204.45125 59.404) (width 0.381) (layer "B.Cu") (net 7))
 (segment (start 203.584842 58.7375) (end 203.598796 58.751454) (width 0.381) (layer "B.Cu") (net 7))
 (segment (start 199.644 58.7375) (end 203.584842 58.7375) (width 0.381) (layer "B.Cu") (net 7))
 (segment (start 207.78125 54.03125) (end 210.60025 54.03125) (width 0.254) (layer "B.Cu") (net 14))
 (segment (start 210.47325 54.03125) (end 210.66125 54.21925) (width 0.254) (layer "B.Cu") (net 14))
 (segment (start 207.78125 56.1565) (end 206.85125 57.0865) (width 0.254) (layer "B.Cu") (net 14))
 (segment (start 207.78125 54.03125) (end 207.78125 56.1565) (width 0.254) (layer "B.Cu") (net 14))
 (segment (start 210.60025 54.03125) (end 210.78825 54.21925) (width 0.254) (layer "B.Cu") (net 14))
 (segment (start 206.85125 57.0865) (end 206.85125 60.18125) (width 0.254) (layer "B.Cu") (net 14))
 (segment (start 205.56925 52.31925) (end 205.58125 52.33125) (width 0.254) (layer "B.Cu") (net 13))
 (segment (start 204.4065 55.5625) (end 206.05125 57.20725) (width 0.254) (layer "B.Cu") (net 13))
 (segment (start 202.53325 52.31925) (end 205.56925 52.31925) (width 0.254) (layer "B.Cu") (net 13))
 (segment (start 205.58125 52.33125) (end 205.2565 52.33125) (width 0.254) (layer "B.Cu") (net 13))
 (segment (start 204.4065 53.18125) (end 204.4065 55.5625) (width 0.254) (layer "B.Cu") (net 13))
 (segment (start 206.05125 57.20725) (end 206.05125 60.18125) (width 0.254) (layer "B.Cu") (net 13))
 (segment (start 205.2565 52.33125) (end 204.4065 53.18125) (width 0.254) (layer "B.Cu") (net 13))
 (segment (start 186.13775 56.09375) (end 186.13775 57.1625) (width 0.381) (layer "B.Cu") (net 6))
 (segment (start 186.13775 57.1625) (end 183.769 59.53125) (width 0.381) (layer "B.Cu") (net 6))
 (segment (start 183.769 59.53125) (end 183.769 65.0875) (width 0.381) (layer "B.Cu") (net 6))
 (segment (start 212.55125 69.88125) (end 215.328 69.88125) (width 0.254) (layer "B.Cu") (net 8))
 (segment (start 215.328 69.88125) (end 215.519 70.07225) (width 0.254) (layer "B.Cu") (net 8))
 (segment (start 193.294 67.48125) (end 193.294 67.46875) (width 0.254) (layer "B.Cu") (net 11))
 (segment (start 188.5315 62.70625) (end 187.73775 63.5) (width 0.254) (layer "B.Cu") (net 11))
 (segment (start 187.73775 63.5) (end 187.73775 65.88125) (width 0.254) (layer "B.Cu") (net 11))
 (segment (start 193.294 67.48125) (end 201.15125 67.48125) (width 0.254) (layer "B.Cu") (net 11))
 (segment (start 188.5315 62.03125) (end 188.5315 62.70625) (width 0.254) (layer "B.Cu") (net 11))
 (segment (start 187.73775 65.88125) (end 189.32525 67.46875) (width 0.254) (layer "B.Cu") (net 11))
 (segment (start 189.32525 67.46875) (end 193.294 67.46875) (width 0.254) (layer "B.Cu") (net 11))
 (segment (start 187.73775 58.7375) (end 188.5315 59.53125) (width 0.2) (layer "B.Cu") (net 12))
 (segment (start 187.73775 56.09375) (end 187.73775 58.7375) (width 0.2) (layer "B.Cu") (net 12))
 (segment (start 188.5315 59.53125) (end 188.5315 60.20625) (width 0.2) (layer "B.Cu") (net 12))
 (segment (start 186.93775 58.752) (end 185.4835 60.20625) (width 0.2) (layer "B.Cu") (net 41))
 (segment (start 186.93775 56.09375) (end 186.93775 58.752) (width 0.2) (layer "B.Cu") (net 41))
 (segment (start 186.944 65.88125) (end 189.344 68.28125) (width 0.254) (layer "B.Cu") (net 17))
 (segment (start 185.4835 62.03125) (end 186.944 63.49175) (width 0.254) (layer "B.Cu") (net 17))
 (segment (start 186.944 63.49175) (end 186.944 65.88125) (width 0.254) (layer "B.Cu") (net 17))
 (segment (start 189.344 68.28125) (end 201.15125 68.28125) (width 0.254) (layer "B.Cu") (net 17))
 (segment (start 193.294 69.85) (end 191.7065 71.4375) (width 0.254) (layer "F.Cu") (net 10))
 (segment (start 193.294 61.11875) (end 193.294 69.85) (width 0.254) (layer "F.Cu") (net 10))
 (via (at 191.7065 71.4375) (size 0.8) (drill 0.4) (layers "F.Cu" "B.Cu") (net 10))
 (via (at 193.294 61.11875) (size 0.8) (drill 0.4) (layers "F.Cu" "B.Cu") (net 10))
 (segment (start 191.7065 71.4375) (end 189.17525 71.4375) (width 0.254) (layer "B.Cu") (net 10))
 (segment (start 193.30225 61.1105) (end 193.294 61.11875) (width 0.254) (layer "B.Cu") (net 10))
 (segment (start 194.8815 61.1105) (end 193.30225 61.1105) (width 0.254) (layer "B.Cu") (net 10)))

